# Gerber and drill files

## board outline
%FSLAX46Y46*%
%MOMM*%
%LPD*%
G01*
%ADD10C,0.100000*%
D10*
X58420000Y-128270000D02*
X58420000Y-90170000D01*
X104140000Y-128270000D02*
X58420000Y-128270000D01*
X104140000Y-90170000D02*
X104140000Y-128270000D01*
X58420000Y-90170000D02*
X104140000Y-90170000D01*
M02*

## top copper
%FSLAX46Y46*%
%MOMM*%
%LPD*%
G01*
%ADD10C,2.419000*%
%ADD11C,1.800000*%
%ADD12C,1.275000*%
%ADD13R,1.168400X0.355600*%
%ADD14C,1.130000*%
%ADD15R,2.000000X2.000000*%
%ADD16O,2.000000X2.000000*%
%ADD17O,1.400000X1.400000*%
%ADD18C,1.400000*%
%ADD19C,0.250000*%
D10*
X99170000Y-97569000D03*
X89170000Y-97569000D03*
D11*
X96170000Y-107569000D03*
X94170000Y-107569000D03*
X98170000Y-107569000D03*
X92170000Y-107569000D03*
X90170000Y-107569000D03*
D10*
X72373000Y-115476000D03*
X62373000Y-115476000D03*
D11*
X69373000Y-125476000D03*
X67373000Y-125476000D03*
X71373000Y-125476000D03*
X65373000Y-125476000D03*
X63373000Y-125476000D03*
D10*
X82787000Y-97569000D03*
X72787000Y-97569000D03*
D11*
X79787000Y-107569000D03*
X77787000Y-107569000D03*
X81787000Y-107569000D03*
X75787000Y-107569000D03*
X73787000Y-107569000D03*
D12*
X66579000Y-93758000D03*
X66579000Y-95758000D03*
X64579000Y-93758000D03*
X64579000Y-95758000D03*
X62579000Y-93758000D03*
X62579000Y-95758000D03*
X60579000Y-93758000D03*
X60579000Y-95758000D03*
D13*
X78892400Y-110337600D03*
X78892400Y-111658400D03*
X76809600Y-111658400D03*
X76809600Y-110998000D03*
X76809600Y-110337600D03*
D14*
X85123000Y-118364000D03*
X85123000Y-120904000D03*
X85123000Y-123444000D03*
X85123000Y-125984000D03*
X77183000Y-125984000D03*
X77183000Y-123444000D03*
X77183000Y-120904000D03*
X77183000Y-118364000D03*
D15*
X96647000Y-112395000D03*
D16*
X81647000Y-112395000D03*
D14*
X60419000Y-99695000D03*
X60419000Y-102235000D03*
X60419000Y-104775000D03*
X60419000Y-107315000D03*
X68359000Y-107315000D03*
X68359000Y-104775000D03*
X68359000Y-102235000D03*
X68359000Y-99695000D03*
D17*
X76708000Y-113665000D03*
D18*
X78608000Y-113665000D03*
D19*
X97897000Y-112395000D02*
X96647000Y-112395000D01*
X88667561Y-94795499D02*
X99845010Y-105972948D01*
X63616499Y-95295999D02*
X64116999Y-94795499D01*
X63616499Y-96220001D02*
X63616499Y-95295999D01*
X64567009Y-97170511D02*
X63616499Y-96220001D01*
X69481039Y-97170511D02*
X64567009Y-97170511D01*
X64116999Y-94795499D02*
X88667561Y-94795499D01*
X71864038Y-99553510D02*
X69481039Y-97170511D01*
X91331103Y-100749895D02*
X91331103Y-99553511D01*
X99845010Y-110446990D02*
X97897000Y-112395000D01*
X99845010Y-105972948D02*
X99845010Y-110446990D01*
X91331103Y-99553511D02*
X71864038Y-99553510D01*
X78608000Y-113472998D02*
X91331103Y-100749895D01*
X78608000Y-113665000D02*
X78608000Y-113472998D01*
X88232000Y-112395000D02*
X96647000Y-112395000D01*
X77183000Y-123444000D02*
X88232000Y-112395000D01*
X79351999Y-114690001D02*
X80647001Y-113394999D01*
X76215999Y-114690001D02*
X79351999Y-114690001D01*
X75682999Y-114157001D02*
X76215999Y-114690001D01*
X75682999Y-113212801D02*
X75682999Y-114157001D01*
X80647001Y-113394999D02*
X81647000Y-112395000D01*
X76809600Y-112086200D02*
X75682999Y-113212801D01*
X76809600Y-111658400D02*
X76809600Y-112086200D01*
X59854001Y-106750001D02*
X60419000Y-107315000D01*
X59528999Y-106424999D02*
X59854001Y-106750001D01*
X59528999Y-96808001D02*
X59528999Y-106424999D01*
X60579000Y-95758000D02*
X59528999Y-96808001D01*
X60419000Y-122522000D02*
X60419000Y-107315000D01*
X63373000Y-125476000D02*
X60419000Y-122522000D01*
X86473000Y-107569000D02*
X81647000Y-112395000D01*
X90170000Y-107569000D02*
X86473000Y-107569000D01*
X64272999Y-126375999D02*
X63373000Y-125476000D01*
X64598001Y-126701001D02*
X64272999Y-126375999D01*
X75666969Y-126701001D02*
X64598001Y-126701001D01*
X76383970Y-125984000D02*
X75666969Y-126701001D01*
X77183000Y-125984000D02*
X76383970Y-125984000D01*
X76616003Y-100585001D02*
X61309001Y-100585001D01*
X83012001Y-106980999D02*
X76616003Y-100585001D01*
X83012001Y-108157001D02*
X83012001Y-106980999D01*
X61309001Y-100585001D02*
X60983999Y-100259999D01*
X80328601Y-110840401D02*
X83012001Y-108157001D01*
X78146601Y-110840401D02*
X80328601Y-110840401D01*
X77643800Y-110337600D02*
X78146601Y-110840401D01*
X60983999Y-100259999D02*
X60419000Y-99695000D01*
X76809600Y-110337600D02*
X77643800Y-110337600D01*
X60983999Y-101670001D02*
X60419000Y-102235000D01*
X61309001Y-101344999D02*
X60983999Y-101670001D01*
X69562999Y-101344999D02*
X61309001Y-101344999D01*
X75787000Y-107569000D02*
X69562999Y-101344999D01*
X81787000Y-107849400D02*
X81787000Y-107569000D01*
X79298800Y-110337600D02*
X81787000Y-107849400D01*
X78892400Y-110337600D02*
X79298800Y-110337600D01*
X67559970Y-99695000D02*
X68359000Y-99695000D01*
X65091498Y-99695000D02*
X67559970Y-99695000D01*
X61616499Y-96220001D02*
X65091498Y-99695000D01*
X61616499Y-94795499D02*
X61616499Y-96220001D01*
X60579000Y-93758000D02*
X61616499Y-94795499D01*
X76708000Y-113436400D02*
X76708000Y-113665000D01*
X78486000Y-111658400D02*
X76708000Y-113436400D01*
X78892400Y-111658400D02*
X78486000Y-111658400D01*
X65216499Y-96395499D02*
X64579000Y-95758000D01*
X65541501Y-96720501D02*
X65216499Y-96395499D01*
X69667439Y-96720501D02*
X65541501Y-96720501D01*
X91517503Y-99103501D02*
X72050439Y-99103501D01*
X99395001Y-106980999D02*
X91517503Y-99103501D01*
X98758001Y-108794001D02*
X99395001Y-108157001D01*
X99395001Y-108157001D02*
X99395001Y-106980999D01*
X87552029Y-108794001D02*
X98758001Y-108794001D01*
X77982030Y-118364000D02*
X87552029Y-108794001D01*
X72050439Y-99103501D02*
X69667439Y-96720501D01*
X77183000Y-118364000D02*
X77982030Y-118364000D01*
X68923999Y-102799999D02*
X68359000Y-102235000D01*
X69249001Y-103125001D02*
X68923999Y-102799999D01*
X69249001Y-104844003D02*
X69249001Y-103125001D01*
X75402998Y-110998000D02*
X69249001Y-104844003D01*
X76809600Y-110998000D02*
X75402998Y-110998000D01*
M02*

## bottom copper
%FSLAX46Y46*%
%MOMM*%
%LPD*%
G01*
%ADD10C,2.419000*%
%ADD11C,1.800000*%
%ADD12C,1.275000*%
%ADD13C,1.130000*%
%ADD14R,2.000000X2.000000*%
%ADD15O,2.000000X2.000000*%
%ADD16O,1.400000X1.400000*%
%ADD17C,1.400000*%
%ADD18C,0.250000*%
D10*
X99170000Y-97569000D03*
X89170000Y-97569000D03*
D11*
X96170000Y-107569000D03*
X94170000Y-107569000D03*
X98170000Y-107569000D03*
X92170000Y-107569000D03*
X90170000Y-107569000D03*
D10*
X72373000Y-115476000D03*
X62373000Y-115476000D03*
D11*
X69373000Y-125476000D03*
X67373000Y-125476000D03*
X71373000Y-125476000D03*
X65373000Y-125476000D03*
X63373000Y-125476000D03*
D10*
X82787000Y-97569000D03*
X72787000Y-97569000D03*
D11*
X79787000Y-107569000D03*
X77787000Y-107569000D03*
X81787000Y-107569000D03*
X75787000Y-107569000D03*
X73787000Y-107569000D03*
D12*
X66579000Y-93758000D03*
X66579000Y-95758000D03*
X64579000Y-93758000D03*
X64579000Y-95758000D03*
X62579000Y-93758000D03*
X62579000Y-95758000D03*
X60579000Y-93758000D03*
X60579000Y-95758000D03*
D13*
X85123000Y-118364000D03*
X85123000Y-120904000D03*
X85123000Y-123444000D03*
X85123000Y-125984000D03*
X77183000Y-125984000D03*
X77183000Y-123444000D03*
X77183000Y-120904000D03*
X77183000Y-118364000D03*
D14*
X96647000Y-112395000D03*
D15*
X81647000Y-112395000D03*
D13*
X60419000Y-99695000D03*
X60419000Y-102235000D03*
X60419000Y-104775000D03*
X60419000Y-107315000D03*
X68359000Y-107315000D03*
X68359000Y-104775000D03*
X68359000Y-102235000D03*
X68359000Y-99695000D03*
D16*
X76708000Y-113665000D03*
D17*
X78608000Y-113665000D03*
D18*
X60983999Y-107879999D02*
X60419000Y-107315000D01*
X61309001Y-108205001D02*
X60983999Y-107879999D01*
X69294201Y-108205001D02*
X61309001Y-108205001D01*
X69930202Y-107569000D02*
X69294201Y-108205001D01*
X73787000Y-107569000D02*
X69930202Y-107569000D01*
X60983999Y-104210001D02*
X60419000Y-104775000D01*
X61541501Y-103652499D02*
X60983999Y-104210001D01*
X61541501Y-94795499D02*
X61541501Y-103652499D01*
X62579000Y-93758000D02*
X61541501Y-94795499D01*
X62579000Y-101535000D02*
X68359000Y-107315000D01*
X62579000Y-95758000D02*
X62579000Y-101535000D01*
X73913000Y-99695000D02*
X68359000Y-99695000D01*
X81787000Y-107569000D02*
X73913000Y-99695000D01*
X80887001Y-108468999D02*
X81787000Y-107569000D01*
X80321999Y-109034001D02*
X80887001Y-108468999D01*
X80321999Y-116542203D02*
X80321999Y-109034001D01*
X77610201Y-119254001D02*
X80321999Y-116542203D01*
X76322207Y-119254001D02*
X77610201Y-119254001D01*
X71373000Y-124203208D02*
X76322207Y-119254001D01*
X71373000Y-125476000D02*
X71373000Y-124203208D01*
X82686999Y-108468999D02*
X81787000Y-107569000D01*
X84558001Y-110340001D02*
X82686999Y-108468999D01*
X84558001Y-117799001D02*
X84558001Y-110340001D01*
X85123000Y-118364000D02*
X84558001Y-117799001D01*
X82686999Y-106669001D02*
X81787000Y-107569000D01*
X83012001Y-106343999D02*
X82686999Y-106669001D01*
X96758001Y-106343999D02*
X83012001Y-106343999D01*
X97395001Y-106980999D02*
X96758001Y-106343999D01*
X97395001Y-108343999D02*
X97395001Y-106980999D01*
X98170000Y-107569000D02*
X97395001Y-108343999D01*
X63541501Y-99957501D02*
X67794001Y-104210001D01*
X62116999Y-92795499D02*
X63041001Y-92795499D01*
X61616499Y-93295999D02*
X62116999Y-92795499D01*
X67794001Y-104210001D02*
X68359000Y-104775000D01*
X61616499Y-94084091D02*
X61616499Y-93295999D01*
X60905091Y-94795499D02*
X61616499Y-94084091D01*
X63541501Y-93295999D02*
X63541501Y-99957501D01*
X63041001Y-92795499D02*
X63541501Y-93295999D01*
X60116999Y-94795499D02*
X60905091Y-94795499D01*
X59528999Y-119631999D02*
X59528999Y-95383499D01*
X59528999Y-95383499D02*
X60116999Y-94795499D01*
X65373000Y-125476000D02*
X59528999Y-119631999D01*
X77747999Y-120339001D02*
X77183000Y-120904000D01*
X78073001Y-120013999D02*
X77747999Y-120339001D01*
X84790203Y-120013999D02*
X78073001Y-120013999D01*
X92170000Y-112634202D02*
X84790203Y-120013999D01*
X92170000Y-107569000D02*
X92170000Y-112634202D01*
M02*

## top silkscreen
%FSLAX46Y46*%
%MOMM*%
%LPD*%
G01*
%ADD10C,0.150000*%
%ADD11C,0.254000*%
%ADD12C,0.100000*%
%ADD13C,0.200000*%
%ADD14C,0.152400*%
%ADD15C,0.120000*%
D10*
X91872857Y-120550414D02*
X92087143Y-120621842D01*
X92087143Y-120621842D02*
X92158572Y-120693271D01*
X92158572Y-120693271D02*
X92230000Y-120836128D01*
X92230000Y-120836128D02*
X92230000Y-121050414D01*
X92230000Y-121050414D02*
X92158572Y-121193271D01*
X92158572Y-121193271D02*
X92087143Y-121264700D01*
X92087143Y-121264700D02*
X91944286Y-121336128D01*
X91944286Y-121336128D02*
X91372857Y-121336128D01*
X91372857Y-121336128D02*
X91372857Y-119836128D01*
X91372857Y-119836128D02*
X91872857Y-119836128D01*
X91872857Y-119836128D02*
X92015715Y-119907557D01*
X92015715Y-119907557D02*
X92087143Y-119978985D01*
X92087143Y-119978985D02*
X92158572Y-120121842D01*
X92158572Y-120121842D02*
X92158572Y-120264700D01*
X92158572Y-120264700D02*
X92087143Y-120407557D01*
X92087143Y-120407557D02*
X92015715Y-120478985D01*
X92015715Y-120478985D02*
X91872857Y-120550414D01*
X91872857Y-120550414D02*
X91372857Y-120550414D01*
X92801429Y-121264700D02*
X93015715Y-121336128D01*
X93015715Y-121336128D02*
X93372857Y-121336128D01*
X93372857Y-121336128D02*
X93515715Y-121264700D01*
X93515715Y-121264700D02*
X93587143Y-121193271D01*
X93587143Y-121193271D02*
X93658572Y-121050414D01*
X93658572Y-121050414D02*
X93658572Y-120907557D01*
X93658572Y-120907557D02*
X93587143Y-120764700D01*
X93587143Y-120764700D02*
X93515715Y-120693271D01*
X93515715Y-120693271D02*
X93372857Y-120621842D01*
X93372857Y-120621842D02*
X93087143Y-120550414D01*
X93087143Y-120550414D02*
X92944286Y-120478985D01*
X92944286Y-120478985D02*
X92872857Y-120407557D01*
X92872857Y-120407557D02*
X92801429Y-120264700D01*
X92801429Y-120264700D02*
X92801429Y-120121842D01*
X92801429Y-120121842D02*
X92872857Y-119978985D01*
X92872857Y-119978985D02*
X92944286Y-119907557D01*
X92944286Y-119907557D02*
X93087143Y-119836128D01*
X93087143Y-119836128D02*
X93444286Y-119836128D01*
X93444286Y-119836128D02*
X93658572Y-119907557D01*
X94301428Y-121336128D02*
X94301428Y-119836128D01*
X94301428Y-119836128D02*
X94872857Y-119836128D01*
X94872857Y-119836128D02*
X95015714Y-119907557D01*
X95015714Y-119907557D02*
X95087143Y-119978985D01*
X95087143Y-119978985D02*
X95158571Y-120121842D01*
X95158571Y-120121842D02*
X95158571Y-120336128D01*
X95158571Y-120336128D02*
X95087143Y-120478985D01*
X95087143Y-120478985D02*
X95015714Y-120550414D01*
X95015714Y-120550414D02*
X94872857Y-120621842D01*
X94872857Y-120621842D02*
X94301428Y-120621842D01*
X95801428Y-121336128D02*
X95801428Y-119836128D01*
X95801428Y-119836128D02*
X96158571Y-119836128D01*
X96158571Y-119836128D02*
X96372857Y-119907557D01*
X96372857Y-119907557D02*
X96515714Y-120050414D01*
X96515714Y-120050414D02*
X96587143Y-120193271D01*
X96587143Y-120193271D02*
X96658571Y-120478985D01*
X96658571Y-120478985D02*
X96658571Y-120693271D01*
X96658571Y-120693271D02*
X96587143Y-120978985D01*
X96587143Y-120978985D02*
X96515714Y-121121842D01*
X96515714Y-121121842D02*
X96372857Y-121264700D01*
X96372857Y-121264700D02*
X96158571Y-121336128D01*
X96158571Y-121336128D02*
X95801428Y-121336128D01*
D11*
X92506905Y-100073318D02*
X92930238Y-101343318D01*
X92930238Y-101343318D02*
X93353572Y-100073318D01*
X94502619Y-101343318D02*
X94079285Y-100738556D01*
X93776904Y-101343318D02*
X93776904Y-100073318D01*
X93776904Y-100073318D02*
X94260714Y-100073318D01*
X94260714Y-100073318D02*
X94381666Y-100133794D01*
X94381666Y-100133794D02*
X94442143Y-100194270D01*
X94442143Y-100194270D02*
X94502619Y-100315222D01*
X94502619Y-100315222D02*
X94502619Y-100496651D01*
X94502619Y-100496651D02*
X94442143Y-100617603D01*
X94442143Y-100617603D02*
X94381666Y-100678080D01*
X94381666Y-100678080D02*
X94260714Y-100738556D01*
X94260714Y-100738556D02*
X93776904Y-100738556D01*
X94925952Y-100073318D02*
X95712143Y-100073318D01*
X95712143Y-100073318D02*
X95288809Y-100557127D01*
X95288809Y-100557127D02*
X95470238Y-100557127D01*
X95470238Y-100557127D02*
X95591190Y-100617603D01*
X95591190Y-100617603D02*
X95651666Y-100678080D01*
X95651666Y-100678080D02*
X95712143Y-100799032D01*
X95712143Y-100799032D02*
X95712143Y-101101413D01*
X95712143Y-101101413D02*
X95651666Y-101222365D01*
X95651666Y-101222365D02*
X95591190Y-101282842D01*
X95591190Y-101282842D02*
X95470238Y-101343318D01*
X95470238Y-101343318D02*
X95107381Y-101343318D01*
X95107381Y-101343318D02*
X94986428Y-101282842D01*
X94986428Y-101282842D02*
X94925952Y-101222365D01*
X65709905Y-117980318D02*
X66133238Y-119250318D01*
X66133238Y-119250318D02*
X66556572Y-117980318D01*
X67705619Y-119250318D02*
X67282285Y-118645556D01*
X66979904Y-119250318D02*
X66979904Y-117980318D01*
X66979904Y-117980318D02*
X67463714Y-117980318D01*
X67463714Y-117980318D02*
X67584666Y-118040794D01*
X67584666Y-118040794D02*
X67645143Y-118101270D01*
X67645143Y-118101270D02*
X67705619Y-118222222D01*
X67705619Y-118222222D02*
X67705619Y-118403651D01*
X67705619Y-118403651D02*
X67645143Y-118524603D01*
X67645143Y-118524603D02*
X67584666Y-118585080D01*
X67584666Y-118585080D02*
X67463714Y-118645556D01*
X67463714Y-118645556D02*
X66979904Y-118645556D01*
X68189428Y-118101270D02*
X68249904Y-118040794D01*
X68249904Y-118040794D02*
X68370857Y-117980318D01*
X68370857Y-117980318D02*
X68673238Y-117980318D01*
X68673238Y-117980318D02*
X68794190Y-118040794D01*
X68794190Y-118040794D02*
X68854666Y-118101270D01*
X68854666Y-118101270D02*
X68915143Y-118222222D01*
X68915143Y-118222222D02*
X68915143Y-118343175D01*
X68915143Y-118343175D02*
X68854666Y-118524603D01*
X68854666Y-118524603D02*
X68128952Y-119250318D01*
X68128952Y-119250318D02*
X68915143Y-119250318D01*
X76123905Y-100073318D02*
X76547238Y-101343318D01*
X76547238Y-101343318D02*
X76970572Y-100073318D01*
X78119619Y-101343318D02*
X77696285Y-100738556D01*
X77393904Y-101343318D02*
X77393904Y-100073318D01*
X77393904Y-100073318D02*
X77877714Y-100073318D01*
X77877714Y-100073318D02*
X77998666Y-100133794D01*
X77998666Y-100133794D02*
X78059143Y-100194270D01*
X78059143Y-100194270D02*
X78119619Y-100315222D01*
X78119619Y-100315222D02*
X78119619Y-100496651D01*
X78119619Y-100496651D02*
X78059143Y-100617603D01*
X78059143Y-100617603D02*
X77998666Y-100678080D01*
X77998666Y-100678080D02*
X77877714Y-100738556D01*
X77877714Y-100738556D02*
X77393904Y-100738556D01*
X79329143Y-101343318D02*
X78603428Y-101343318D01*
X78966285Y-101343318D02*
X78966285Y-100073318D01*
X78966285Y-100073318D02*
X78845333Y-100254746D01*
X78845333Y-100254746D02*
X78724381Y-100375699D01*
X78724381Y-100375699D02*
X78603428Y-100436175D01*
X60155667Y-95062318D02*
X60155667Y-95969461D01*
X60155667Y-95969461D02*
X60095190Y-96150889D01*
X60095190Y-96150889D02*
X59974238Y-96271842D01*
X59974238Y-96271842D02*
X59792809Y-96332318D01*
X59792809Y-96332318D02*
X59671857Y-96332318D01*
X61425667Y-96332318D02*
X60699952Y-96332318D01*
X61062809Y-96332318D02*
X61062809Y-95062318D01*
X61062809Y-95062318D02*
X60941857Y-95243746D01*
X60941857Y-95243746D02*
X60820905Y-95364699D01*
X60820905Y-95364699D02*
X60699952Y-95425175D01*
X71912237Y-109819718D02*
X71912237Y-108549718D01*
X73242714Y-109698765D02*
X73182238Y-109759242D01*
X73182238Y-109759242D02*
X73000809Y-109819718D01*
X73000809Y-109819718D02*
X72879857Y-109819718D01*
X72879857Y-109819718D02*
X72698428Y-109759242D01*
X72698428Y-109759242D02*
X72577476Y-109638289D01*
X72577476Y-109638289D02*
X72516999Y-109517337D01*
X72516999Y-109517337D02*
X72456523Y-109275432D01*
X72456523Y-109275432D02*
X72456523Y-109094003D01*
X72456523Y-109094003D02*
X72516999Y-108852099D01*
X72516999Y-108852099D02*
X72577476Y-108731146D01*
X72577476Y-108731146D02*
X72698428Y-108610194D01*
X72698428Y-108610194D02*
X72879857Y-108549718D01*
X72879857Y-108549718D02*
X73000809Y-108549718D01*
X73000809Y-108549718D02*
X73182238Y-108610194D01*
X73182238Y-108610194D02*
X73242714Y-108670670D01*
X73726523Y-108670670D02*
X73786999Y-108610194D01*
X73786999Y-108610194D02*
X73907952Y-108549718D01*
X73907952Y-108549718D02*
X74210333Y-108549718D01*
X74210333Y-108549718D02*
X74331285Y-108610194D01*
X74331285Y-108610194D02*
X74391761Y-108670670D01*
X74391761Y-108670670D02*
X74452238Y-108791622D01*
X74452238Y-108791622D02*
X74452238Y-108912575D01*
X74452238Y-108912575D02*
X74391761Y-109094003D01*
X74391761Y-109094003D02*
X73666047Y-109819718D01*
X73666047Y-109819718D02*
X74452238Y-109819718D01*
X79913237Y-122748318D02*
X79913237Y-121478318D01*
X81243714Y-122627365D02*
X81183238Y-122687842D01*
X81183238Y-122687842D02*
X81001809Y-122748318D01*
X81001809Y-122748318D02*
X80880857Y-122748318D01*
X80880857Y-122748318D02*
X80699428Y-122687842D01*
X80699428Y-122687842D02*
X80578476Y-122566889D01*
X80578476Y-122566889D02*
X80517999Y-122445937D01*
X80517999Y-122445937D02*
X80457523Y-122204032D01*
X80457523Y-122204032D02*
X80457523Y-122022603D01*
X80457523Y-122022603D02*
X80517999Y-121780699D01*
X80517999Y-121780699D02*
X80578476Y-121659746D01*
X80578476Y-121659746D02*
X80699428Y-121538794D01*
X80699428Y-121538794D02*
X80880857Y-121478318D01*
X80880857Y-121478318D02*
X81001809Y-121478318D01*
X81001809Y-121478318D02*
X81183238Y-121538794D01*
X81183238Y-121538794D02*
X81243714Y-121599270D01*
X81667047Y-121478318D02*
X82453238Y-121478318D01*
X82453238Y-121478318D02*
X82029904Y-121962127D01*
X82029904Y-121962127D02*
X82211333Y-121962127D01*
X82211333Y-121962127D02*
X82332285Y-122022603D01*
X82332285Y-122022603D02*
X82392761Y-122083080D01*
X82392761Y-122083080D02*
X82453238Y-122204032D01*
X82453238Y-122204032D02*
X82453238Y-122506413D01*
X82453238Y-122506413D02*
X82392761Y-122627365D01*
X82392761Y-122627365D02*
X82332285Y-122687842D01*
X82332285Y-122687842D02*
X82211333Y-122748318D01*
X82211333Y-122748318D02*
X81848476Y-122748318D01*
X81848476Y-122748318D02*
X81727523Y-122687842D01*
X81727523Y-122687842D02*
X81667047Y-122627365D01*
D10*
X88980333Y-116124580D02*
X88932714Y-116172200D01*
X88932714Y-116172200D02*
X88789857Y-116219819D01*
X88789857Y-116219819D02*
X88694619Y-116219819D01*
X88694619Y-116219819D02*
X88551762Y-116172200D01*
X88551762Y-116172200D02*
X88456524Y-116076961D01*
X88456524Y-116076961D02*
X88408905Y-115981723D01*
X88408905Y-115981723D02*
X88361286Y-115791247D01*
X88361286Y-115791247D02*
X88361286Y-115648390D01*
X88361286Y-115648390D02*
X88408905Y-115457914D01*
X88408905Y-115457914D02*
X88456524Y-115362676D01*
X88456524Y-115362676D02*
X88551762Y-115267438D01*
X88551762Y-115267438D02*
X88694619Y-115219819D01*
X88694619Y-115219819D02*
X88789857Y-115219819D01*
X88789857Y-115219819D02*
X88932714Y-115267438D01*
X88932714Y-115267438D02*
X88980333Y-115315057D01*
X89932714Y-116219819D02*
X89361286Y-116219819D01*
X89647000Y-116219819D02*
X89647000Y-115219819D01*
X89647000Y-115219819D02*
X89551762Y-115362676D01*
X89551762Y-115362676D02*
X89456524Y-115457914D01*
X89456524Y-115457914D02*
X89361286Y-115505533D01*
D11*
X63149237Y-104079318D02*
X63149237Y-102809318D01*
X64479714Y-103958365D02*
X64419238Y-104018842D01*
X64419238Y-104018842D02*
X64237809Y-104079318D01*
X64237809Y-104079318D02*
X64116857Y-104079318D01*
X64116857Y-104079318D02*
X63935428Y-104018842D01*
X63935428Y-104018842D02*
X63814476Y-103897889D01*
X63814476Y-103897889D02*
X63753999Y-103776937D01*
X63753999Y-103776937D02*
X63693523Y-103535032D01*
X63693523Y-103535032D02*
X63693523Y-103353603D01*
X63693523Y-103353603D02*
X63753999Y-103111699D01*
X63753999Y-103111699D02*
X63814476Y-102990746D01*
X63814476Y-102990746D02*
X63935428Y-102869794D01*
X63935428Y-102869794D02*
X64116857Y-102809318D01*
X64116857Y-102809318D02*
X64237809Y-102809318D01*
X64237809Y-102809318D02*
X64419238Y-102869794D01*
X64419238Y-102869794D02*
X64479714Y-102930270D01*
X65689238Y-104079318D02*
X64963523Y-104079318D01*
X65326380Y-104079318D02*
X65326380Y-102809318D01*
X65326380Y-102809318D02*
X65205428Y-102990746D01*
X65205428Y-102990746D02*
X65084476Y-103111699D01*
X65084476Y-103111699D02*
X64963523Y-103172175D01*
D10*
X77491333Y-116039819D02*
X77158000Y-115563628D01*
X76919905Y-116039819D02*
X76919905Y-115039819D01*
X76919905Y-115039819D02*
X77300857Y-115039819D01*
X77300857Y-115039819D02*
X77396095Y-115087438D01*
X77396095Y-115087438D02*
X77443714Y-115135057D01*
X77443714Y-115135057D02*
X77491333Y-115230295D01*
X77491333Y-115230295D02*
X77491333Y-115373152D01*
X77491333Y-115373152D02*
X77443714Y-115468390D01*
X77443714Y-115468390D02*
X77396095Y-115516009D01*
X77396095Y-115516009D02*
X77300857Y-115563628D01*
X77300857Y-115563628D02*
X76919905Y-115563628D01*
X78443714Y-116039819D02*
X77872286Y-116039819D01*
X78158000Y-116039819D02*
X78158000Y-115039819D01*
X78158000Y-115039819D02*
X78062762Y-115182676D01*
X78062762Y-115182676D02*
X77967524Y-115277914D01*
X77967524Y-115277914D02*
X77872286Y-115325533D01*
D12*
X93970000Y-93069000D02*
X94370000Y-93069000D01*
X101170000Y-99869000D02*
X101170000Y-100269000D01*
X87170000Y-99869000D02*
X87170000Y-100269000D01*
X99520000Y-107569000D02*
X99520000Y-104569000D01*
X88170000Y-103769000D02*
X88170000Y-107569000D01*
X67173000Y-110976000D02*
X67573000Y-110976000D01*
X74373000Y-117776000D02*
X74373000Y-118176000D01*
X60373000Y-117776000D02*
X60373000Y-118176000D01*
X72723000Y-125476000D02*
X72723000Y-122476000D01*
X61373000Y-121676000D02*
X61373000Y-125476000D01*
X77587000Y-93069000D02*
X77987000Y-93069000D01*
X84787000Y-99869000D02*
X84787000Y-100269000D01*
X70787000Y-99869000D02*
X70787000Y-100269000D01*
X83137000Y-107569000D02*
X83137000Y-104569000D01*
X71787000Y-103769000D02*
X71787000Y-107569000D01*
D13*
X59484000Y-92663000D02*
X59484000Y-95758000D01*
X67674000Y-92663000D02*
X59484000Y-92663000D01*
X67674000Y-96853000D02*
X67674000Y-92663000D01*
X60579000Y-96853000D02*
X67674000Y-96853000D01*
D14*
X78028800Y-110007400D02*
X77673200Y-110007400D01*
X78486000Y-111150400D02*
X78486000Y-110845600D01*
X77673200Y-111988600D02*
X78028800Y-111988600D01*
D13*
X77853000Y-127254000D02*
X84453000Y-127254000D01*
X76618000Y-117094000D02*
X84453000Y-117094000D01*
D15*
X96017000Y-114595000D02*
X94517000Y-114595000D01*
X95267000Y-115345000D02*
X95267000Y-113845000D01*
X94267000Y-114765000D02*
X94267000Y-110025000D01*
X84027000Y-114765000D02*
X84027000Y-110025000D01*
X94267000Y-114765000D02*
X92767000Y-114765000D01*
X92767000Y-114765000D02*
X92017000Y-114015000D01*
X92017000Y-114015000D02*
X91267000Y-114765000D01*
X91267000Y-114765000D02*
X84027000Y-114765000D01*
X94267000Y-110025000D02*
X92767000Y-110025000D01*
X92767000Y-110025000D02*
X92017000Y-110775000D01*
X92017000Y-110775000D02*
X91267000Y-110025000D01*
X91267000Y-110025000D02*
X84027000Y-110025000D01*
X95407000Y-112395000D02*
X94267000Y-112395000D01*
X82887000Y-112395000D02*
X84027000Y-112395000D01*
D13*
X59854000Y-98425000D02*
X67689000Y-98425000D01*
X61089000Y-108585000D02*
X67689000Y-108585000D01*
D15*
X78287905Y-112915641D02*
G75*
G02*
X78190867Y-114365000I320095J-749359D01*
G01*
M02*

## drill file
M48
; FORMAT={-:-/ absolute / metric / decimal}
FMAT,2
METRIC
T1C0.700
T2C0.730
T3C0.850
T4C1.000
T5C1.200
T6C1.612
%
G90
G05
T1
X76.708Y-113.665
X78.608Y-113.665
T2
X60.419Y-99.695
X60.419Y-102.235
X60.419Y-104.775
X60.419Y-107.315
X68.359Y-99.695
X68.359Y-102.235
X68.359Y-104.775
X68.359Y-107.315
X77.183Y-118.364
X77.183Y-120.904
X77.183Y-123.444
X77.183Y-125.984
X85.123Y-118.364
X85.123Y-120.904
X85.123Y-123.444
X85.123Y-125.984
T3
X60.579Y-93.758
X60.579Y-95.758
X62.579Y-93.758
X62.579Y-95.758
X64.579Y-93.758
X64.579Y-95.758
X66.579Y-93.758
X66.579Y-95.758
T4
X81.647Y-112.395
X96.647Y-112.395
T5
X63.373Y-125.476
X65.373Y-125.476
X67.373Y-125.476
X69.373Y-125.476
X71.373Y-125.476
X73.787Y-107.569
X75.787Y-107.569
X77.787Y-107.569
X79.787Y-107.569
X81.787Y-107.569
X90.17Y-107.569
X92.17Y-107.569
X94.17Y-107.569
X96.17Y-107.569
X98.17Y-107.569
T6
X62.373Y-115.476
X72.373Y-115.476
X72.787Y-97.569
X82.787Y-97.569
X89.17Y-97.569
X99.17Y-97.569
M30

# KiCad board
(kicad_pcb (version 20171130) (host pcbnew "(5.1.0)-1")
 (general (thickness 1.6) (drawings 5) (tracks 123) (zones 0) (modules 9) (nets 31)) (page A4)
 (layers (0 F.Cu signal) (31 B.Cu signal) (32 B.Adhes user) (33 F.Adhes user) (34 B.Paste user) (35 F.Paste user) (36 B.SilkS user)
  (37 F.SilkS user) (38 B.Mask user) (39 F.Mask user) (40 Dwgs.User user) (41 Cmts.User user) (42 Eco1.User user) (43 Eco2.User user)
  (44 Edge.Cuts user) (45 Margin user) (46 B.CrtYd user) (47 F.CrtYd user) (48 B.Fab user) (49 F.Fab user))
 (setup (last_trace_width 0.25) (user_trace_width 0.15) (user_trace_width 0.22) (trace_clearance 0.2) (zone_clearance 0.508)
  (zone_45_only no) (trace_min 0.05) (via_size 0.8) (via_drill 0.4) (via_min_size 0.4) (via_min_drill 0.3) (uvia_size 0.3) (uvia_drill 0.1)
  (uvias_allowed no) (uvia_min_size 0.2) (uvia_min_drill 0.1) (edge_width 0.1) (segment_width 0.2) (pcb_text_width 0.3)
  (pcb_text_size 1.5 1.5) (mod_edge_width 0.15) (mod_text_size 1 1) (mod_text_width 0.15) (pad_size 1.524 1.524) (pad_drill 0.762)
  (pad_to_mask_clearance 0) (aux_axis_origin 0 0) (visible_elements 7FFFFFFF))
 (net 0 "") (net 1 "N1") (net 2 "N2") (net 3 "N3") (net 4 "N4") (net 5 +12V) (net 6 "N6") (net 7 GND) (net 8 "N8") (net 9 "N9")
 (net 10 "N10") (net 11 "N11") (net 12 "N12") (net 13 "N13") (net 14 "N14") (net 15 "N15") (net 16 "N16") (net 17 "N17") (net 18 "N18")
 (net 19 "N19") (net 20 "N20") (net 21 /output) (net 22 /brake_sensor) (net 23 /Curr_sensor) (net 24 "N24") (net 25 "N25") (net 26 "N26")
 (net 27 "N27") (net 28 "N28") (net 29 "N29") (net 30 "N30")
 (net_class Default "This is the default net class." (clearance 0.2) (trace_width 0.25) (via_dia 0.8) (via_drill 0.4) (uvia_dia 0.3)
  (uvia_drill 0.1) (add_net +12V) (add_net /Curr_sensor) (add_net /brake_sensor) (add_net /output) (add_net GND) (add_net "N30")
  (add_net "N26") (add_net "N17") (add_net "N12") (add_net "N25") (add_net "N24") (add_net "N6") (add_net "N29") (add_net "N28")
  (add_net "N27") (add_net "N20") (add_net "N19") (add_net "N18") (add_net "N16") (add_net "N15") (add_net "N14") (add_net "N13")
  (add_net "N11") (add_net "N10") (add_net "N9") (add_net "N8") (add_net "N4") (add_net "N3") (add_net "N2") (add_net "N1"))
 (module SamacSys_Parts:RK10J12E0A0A (layer F.Cu) (at 90.17 107.569)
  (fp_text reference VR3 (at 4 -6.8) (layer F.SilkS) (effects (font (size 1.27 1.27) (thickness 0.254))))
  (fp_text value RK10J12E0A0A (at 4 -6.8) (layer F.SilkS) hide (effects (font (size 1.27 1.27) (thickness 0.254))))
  (fp_line (start 3.8 -14.5) (end 4.2 -14.5) (layer F.SilkS) (width 0.1))
  (fp_line (start 11 -7.7) (end 11 -7.3) (layer F.SilkS) (width 0.1))
  (fp_line (start -3 -7.7) (end -3 -7.3) (layer F.SilkS) (width 0.1))
  (fp_line (start 9.35 0) (end 9.35 -3) (layer F.SilkS) (width 0.1))
  (fp_line (start -2 -3.8) (end -2 0) (layer F.SilkS) (width 0.1))
  (pad MH2 thru_hole circle (at 9 -10) (size 2.419 2.419) (drill 1.6125) (layers *.Cu *.Mask) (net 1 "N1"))
  (pad MH1 thru_hole circle (at -1 -10) (size 2.419 2.419) (drill 1.6125) (layers *.Cu *.Mask) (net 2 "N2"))
  (pad 5 thru_hole circle (at 6 0) (size 1.8 1.8) (drill 1.2) (layers *.Cu *.Mask) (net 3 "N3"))
  (pad 4 thru_hole circle (at 4 0) (size 1.8 1.8) (drill 1.2) (layers *.Cu *.Mask) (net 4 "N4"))
  (pad 3 thru_hole circle (at 8 0) (size 1.8 1.8) (drill 1.2) (layers *.Cu *.Mask) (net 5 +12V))
  (pad 2 thru_hole circle (at 2 0) (size 1.8 1.8) (drill 1.2) (layers *.Cu *.Mask) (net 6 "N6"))
  (pad 1 thru_hole circle (at 0 0) (size 1.8 1.8) (drill 1.2) (layers *.Cu *.Mask) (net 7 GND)))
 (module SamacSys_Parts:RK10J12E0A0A (layer F.Cu) (at 63.373 125.476)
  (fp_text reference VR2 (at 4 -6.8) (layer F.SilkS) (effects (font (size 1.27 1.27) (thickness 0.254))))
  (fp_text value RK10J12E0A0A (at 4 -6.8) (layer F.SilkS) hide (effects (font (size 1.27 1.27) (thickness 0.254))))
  (fp_line (start 3.8 -14.5) (end 4.2 -14.5) (layer F.SilkS) (width 0.1))
  (fp_line (start 11 -7.7) (end 11 -7.3) (layer F.SilkS) (width 0.1))
  (fp_line (start -3 -7.7) (end -3 -7.3) (layer F.SilkS) (width 0.1))
  (fp_line (start 9.35 0) (end 9.35 -3) (layer F.SilkS) (width 0.1))
  (fp_line (start -2 -3.8) (end -2 0) (layer F.SilkS) (width 0.1))
  (pad MH2 thru_hole circle (at 9 -10) (size 2.419 2.419) (drill 1.6125) (layers *.Cu *.Mask) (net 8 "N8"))
  (pad MH1 thru_hole circle (at -1 -10) (size 2.419 2.419) (drill 1.6125) (layers *.Cu *.Mask) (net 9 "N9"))
  (pad 5 thru_hole circle (at 6 0) (size 1.8 1.8) (drill 1.2) (layers *.Cu *.Mask) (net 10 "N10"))
  (pad 4 thru_hole circle (at 4 0) (size 1.8 1.8) (drill 1.2) (layers *.Cu *.Mask) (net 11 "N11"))
  (pad 3 thru_hole circle (at 8 0) (size 1.8 1.8) (drill 1.2) (layers *.Cu *.Mask) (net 5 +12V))
  (pad 2 thru_hole circle (at 2 0) (size 1.8 1.8) (drill 1.2) (layers *.Cu *.Mask) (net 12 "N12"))
  (pad 1 thru_hole circle (at 0 0) (size 1.8 1.8) (drill 1.2) (layers *.Cu *.Mask) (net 7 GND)))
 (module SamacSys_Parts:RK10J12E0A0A (layer F.Cu) (at 73.787 107.569)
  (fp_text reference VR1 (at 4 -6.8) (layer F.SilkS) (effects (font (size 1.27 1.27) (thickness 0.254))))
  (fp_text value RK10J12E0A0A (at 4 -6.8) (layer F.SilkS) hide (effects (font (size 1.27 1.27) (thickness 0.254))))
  (fp_line (start 3.8 -14.5) (end 4.2 -14.5) (layer F.SilkS) (width 0.1))
  (fp_line (start 11 -7.7) (end 11 -7.3) (layer F.SilkS) (width 0.1))
  (fp_line (start -3 -7.7) (end -3 -7.3) (layer F.SilkS) (width 0.1))
  (fp_line (start 9.35 0) (end 9.35 -3) (layer F.SilkS) (width 0.1))
  (fp_line (start -2 -3.8) (end -2 0) (layer F.SilkS) (width 0.1))
  (pad MH2 thru_hole circle (at 9 -10) (size 2.419 2.419) (drill 1.6125) (layers *.Cu *.Mask) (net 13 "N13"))
  (pad MH1 thru_hole circle (at -1 -10) (size 2.419 2.419) (drill 1.6125) (layers *.Cu *.Mask) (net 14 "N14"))
  (pad 5 thru_hole circle (at 6 0) (size 1.8 1.8) (drill 1.2) (layers *.Cu *.Mask) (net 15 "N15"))
  (pad 4 thru_hole circle (at 4 0) (size 1.8 1.8) (drill 1.2) (layers *.Cu *.Mask) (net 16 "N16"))
  (pad 3 thru_hole circle (at 8 0) (size 1.8 1.8) (drill 1.2) (layers *.Cu *.Mask) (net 5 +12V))
  (pad 2 thru_hole circle (at 2 0) (size 1.8 1.8) (drill 1.2) (layers *.Cu *.Mask) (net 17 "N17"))
  (pad 1 thru_hole circle (at 0 0) (size 1.8 1.8) (drill 1.2) (layers *.Cu *.Mask) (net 7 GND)))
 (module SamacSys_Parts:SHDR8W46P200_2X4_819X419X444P (layer F.Cu) (at 60.579 95.758)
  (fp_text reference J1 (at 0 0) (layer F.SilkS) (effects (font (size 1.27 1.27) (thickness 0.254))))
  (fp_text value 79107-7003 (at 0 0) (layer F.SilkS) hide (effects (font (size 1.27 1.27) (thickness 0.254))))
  (fp_line (start -1.095 -3.095) (end -1.095 0) (layer F.SilkS) (width 0.2))
  (fp_line (start 7.095 -3.095) (end -1.095 -3.095) (layer F.SilkS) (width 0.2))
  (fp_line (start 7.095 1.095) (end 7.095 -3.095) (layer F.SilkS) (width 0.2))
  (fp_line (start 0 1.095) (end 7.095 1.095) (layer F.SilkS) (width 0.2))
  (pad 8 thru_hole circle (at 6 -2) (size 1.275 1.275) (drill 0.85) (layers *.Cu *.Mask) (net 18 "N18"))
  (pad 7 thru_hole circle (at 6 0) (size 1.275 1.275) (drill 0.85) (layers *.Cu *.Mask) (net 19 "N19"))
  (pad 6 thru_hole circle (at 4 -2) (size 1.275 1.275) (drill 0.85) (layers *.Cu *.Mask) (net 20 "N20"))
  (pad 5 thru_hole circle (at 4 0) (size 1.275 1.275) (drill 0.85) (layers *.Cu *.Mask) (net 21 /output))
  (pad 4 thru_hole circle (at 2 -2) (size 1.275 1.275) (drill 0.85) (layers *.Cu *.Mask) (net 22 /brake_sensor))
  (pad 3 thru_hole circle (at 2 0) (size 1.275 1.275) (drill 0.85) (layers *.Cu *.Mask) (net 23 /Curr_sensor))
  (pad 2 thru_hole circle (at 0 -2) (size 1.275 1.275) (drill 0.85) (layers *.Cu *.Mask) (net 5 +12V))
  (pad 1 thru_hole circle (at 0 0) (size 1.275 1.275) (drill 0.85) (layers *.Cu *.Mask) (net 7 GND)))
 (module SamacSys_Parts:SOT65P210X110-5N (layer F.Cu) (at 77.851 110.998)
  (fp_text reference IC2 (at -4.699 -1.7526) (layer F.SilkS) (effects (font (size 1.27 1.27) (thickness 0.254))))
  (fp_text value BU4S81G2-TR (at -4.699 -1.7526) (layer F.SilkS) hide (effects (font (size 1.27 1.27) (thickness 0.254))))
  (fp_line (start 0.1778 -0.9906) (end -0.1778 -0.9906) (layer F.SilkS) (width 0.1524))
  (fp_line (start 0.635 0.1524) (end 0.635 -0.1524) (layer F.SilkS) (width 0.1524))
  (fp_line (start -0.1778 0.9906) (end 0.1778 0.9906) (layer F.SilkS) (width 0.1524))
  (pad 5 smd rect (at 1.0414 -0.6604 90) (size 0.3556 1.1684) (layers F.Cu F.Paste F.Mask) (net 5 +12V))
  (pad 4 smd rect (at 1.0414 0.6604 90) (size 0.3556 1.1684) (layers F.Cu F.Paste F.Mask) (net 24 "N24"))
  (pad 3 smd rect (at -1.0414 0.6604 90) (size 0.3556 1.1684) (layers F.Cu F.Paste F.Mask) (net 7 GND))
  (pad 2 smd rect (at -1.0414 0 90) (size 0.3556 1.1684) (layers F.Cu F.Paste F.Mask) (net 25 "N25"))
  (pad 1 smd rect (at -1.0414 -0.6604 90) (size 0.3556 1.1684) (layers F.Cu F.Paste F.Mask) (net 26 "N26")))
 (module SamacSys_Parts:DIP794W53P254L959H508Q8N (layer F.Cu) (at 81.153 122.174)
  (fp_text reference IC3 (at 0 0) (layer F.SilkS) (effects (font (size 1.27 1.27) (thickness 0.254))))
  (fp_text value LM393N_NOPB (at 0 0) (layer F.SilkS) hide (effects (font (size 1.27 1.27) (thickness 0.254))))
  (fp_line (start -3.3 5.08) (end 3.3 5.08) (layer F.SilkS) (width 0.2))
  (fp_line (start -4.535 -5.08) (end 3.3 -5.08) (layer F.SilkS) (width 0.2))
  (pad 8 thru_hole circle (at 3.97 -3.81) (size 1.13 1.13) (drill 0.73) (layers *.Cu *.Mask) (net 5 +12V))
  (pad 7 thru_hole circle (at 3.97 -1.27) (size 1.13 1.13) (drill 0.73) (layers *.Cu *.Mask) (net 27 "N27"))
  (pad 6 thru_hole circle (at 3.97 1.27) (size 1.13 1.13) (drill 0.73) (layers *.Cu *.Mask) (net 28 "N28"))
  (pad 5 thru_hole circle (at 3.97 3.81) (size 1.13 1.13) (drill 0.73) (layers *.Cu *.Mask) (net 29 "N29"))
  (pad 4 thru_hole circle (at -3.97 3.81) (size 1.13 1.13) (drill 0.73) (layers *.Cu *.Mask) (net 7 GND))
  (pad 3 thru_hole circle (at -3.97 1.27) (size 1.13 1.13) (drill 0.73) (layers *.Cu *.Mask) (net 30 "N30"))
  (pad 2 thru_hole circle (at -3.97 -1.27) (size 1.13 1.13) (drill 0.73) (layers *.Cu *.Mask) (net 6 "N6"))
  (pad 1 thru_hole circle (at -3.97 -3.81) (size 1.13 1.13) (drill 0.73) (layers *.Cu *.Mask) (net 21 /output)))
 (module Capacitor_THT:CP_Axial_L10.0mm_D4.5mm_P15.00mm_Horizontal (layer F.Cu) (at 96.647 112.395 180)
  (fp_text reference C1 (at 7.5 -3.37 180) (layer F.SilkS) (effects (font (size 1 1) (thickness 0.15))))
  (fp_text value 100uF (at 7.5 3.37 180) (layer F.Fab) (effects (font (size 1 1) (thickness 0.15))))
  (fp_line (start 0.63 -2.2) (end 2.13 -2.2) (layer F.SilkS) (width 0.12))
  (fp_line (start 1.38 -2.95) (end 1.38 -1.45) (layer F.SilkS) (width 0.12))
  (fp_line (start 2.38 -2.37) (end 2.38 2.37) (layer F.SilkS) (width 0.12))
  (fp_line (start 12.62 -2.37) (end 12.62 2.37) (layer F.SilkS) (width 0.12))
  (fp_line (start 2.38 -2.37) (end 3.88 -2.37) (layer F.SilkS) (width 0.12))
  (fp_line (start 3.88 -2.37) (end 4.63 -1.62) (layer F.SilkS) (width 0.12))
  (fp_line (start 4.63 -1.62) (end 5.38 -2.37) (layer F.SilkS) (width 0.12))
  (fp_line (start 5.38 -2.37) (end 12.62 -2.37) (layer F.SilkS) (width 0.12))
  (fp_line (start 2.38 2.37) (end 3.88 2.37) (layer F.SilkS) (width 0.12))
  (fp_line (start 3.88 2.37) (end 4.63 1.62) (layer F.SilkS) (width 0.12))
  (fp_line (start 4.63 1.62) (end 5.38 2.37) (layer F.SilkS) (width 0.12))
  (fp_line (start 5.38 2.37) (end 12.62 2.37) (layer F.SilkS) (width 0.12))
  (fp_line (start 1.24 0) (end 2.38 0) (layer F.SilkS) (width 0.12))
  (fp_line (start 13.76 0) (end 12.62 0) (layer F.SilkS) (width 0.12))
  (pad 1 thru_hole rect (at 0 0 180) (size 2 2) (drill 1) (layers *.Cu *.Mask) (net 30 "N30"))
  (pad 2 thru_hole oval (at 15 0 180) (size 2 2) (drill 1) (layers *.Cu *.Mask) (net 7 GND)))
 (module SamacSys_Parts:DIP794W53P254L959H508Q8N (layer F.Cu) (at 64.389 103.505)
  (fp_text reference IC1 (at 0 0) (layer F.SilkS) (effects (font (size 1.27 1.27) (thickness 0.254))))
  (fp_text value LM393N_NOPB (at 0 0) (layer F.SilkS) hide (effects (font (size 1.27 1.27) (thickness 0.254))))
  (fp_line (start -4.535 -5.08) (end 3.3 -5.08) (layer F.SilkS) (width 0.2))
  (fp_line (start -3.3 5.08) (end 3.3 5.08) (layer F.SilkS) (width 0.2))
  (pad 1 thru_hole circle (at -3.97 -3.81) (size 1.13 1.13) (drill 0.73) (layers *.Cu *.Mask) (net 26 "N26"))
  (pad 2 thru_hole circle (at -3.97 -1.27) (size 1.13 1.13) (drill 0.73) (layers *.Cu *.Mask) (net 17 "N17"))
  (pad 3 thru_hole circle (at -3.97 1.27) (size 1.13 1.13) (drill 0.73) (layers *.Cu *.Mask) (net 22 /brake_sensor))
  (pad 4 thru_hole circle (at -3.97 3.81) (size 1.13 1.13) (drill 0.73) (layers *.Cu *.Mask) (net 7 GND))
  (pad 5 thru_hole circle (at 3.97 3.81) (size 1.13 1.13) (drill 0.73) (layers *.Cu *.Mask) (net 23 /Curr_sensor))
  (pad 6 thru_hole circle (at 3.97 1.27) (size 1.13 1.13) (drill 0.73) (layers *.Cu *.Mask) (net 12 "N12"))
  (pad 7 thru_hole circle (at 3.97 -1.27) (size 1.13 1.13) (drill 0.73) (layers *.Cu *.Mask) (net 25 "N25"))
  (pad 8 thru_hole circle (at 3.97 -3.81) (size 1.13 1.13) (drill 0.73) (layers *.Cu *.Mask) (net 5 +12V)))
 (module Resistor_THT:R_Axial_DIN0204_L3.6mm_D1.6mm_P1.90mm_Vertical (layer F.Cu) (at 78.608 113.665 180)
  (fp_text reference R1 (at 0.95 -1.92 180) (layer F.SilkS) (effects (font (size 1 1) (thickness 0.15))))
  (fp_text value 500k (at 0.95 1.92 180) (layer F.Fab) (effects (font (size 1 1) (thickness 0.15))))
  (fp_arc (start 0 0) (end 0.417133 -0.7) (angle -233.92106) (layer F.SilkS) (width 0.12))
  (pad 2 thru_hole oval (at 1.9 0 180) (size 1.4 1.4) (drill 0.7) (layers *.Cu *.Mask) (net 24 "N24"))
  (pad 1 thru_hole circle (at 0 0 180) (size 1.4 1.4) (drill 0.7) (layers *.Cu *.Mask) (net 30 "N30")))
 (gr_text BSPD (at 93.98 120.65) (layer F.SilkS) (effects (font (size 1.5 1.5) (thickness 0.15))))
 (gr_line (start 58.42 128.27) (end 58.42 90.17) (layer Edge.Cuts) (width 0.1))
 (gr_line (start 104.14 128.27) (end 58.42 128.27) (layer Edge.Cuts) (width 0.1))
 (gr_line (start 104.14 90.17) (end 104.14 128.27) (layer Edge.Cuts) (width 0.1))
 (gr_line (start 58.42 90.17) (end 104.14 90.17) (layer Edge.Cuts) (width 0.1))
 (segment (start 97.897 112.395) (end 96.647 112.395) (width 0.25) (layer F.Cu) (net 30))
 (segment (start 88.667561 94.795499) (end 99.84501 105.972948) (width 0.25) (layer F.Cu) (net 30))
 (segment (start 63.616499 95.295999) (end 64.116999 94.795499) (width 0.25) (layer F.Cu) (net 30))
 (segment (start 63.616499 96.220001) (end 63.616499 95.295999) (width 0.25) (layer F.Cu) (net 30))
 (segment (start 64.567009 97.170511) (end 63.616499 96.220001) (width 0.25) (layer F.Cu) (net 30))
 (segment (start 69.481039 97.170511) (end 64.567009 97.170511) (width 0.25) (layer F.Cu) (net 30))
 (segment (start 64.116999 94.795499) (end 88.667561 94.795499) (width 0.25) (layer F.Cu) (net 30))
 (segment (start 71.864038 99.55351) (end 69.481039 97.170511) (width 0.25) (layer F.Cu) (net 30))
 (segment (start 91.331103 100.749895) (end 91.331103 99.553511) (width 0.25) (layer F.Cu) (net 30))
 (segment (start 99.84501 110.44699) (end 97.897 112.395) (width 0.25) (layer F.Cu) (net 30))
 (segment (start 99.84501 105.972948) (end 99.84501 110.44699) (width 0.25) (layer F.Cu) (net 30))
 (segment (start 91.331103 99.553511) (end 71.864038 99.55351) (width 0.25) (layer F.Cu) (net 30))
 (segment (start 78.608 113.472998) (end 91.331103 100.749895) (width 0.25) (layer F.Cu) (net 30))
 (segment (start 78.608 113.665) (end 78.608 113.472998) (width 0.25) (layer F.Cu) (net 30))
 (segment (start 88.232 112.395) (end 96.647 112.395) (width 0.25) (layer F.Cu) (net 30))
 (segment (start 77.183 123.444) (end 88.232 112.395) (width 0.25) (layer F.Cu) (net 30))
 (segment (start 79.351999 114.690001) (end 80.647001 113.394999) (width 0.25) (layer F.Cu) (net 7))
 (segment (start 76.215999 114.690001) (end 79.351999 114.690001) (width 0.25) (layer F.Cu) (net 7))
 (segment (start 75.682999 114.157001) (end 76.215999 114.690001) (width 0.25) (layer F.Cu) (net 7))
 (segment (start 75.682999 113.212801) (end 75.682999 114.157001) (width 0.25) (layer F.Cu) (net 7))
 (segment (start 80.647001 113.394999) (end 81.647 112.395) (width 0.25) (layer F.Cu) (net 7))
 (segment (start 76.8096 112.0862) (end 75.682999 113.212801) (width 0.25) (layer F.Cu) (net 7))
 (segment (start 76.8096 111.6584) (end 76.8096 112.0862) (width 0.25) (layer F.Cu) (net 7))
 (segment (start 59.854001 106.750001) (end 60.419 107.315) (width 0.25) (layer F.Cu) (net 7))
 (segment (start 59.528999 106.424999) (end 59.854001 106.750001) (width 0.25) (layer F.Cu) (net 7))
 (segment (start 59.528999 96.808001) (end 59.528999 106.424999) (width 0.25) (layer F.Cu) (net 7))
 (segment (start 60.579 95.758) (end 59.528999 96.808001) (width 0.25) (layer F.Cu) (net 7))
 (segment (start 60.983999 107.879999) (end 60.419 107.315) (width 0.25) (layer B.Cu) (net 7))
 (segment (start 61.309001 108.205001) (end 60.983999 107.879999) (width 0.25) (layer B.Cu) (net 7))
 (segment (start 69.294201 108.205001) (end 61.309001 108.205001) (width 0.25) (layer B.Cu) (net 7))
 (segment (start 69.930202 107.569) (end 69.294201 108.205001) (width 0.25) (layer B.Cu) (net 7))
 (segment (start 73.787 107.569) (end 69.930202 107.569) (width 0.25) (layer B.Cu) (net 7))
 (segment (start 60.419 122.522) (end 60.419 107.315) (width 0.25) (layer F.Cu) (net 7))
 (segment (start 63.373 125.476) (end 60.419 122.522) (width 0.25) (layer F.Cu) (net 7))
 (segment (start 86.473 107.569) (end 81.647 112.395) (width 0.25) (layer F.Cu) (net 7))
 (segment (start 90.17 107.569) (end 86.473 107.569) (width 0.25) (layer F.Cu) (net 7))
 (segment (start 64.272999 126.375999) (end 63.373 125.476) (width 0.25) (layer F.Cu) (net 7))
 (segment (start 64.598001 126.701001) (end 64.272999 126.375999) (width 0.25) (layer F.Cu) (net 7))
 (segment (start 75.666969 126.701001) (end 64.598001 126.701001) (width 0.25) (layer F.Cu) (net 7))
 (segment (start 76.38397 125.984) (end 75.666969 126.701001) (width 0.25) (layer F.Cu) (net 7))
 (segment (start 77.183 125.984) (end 76.38397 125.984) (width 0.25) (layer F.Cu) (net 7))
 (segment (start 76.616003 100.585001) (end 61.309001 100.585001) (width 0.25) (layer F.Cu) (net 26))
 (segment (start 83.012001 106.980999) (end 76.616003 100.585001) (width 0.25) (layer F.Cu) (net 26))
 (segment (start 83.012001 108.157001) (end 83.012001 106.980999) (width 0.25) (layer F.Cu) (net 26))
 (segment (start 61.309001 100.585001) (end 60.983999 100.259999) (width 0.25) (layer F.Cu) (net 26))
 (segment (start 80.328601 110.840401) (end 83.012001 108.157001) (width 0.25) (layer F.Cu) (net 26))
 (segment (start 78.146601 110.840401) (end 80.328601 110.840401) (width 0.25) (layer F.Cu) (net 26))
 (segment (start 77.6438 110.3376) (end 78.146601 110.840401) (width 0.25) (layer F.Cu) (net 26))
 (segment (start 60.983999 100.259999) (end 60.419 99.695) (width 0.25) (layer F.Cu) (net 26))
 (segment (start 76.8096 110.3376) (end 77.6438 110.3376) (width 0.25) (layer F.Cu) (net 26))
 (segment (start 60.983999 101.670001) (end 60.419 102.235) (width 0.25) (layer F.Cu) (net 17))
 (segment (start 61.309001 101.344999) (end 60.983999 101.670001) (width 0.25) (layer F.Cu) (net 17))
 (segment (start 69.562999 101.344999) (end 61.309001 101.344999) (width 0.25) (layer F.Cu) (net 17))
 (segment (start 75.787 107.569) (end 69.562999 101.344999) (width 0.25) (layer F.Cu) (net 17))
 (segment (start 60.983999 104.210001) (end 60.419 104.775) (width 0.25) (layer B.Cu) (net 22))
 (segment (start 61.541501 103.652499) (end 60.983999 104.210001) (width 0.25) (layer B.Cu) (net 22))
 (segment (start 61.541501 94.795499) (end 61.541501 103.652499) (width 0.25) (layer B.Cu) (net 22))
 (segment (start 62.579 93.758) (end 61.541501 94.795499) (width 0.25) (layer B.Cu) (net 22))
 (segment (start 62.579 101.535) (end 68.359 107.315) (width 0.25) (layer B.Cu) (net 23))
 (segment (start 62.579 95.758) (end 62.579 101.535) (width 0.25) (layer B.Cu) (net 23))
 (segment (start 81.787 107.8494) (end 81.787 107.569) (width 0.25) (layer F.Cu) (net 5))
 (segment (start 79.2988 110.3376) (end 81.787 107.8494) (width 0.25) (layer F.Cu) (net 5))
 (segment (start 78.8924 110.3376) (end 79.2988 110.3376) (width 0.25) (layer F.Cu) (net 5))
 (segment (start 67.55997 99.695) (end 68.359 99.695) (width 0.25) (layer F.Cu) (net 5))
 (segment (start 65.091498 99.695) (end 67.55997 99.695) (width 0.25) (layer F.Cu) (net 5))
 (segment (start 61.616499 96.220001) (end 65.091498 99.695) (width 0.25) (layer F.Cu) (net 5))
 (segment (start 61.616499 94.795499) (end 61.616499 96.220001) (width 0.25) (layer F.Cu) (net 5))
 (segment (start 60.579 93.758) (end 61.616499 94.795499) (width 0.25) (layer F.Cu) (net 5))
 (segment (start 73.913 99.695) (end 68.359 99.695) (width 0.25) (layer B.Cu) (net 5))
 (segment (start 81.787 107.569) (end 73.913 99.695) (width 0.25) (layer B.Cu) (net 5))
 (segment (start 80.887001 108.468999) (end 81.787 107.569) (width 0.25) (layer B.Cu) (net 5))
 (segment (start 80.321999 109.034001) (end 80.887001 108.468999) (width 0.25) (layer B.Cu) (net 5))
 (segment (start 80.321999 116.542203) (end 80.321999 109.034001) (width 0.25) (layer B.Cu) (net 5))
 (segment (start 77.610201 119.254001) (end 80.321999 116.542203) (width 0.25) (layer B.Cu) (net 5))
 (segment (start 76.322207 119.254001) (end 77.610201 119.254001) (width 0.25) (layer B.Cu) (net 5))
 (segment (start 71.373 124.203208) (end 76.322207 119.254001) (width 0.25) (layer B.Cu) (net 5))
 (segment (start 71.373 125.476) (end 71.373 124.203208) (width 0.25) (layer B.Cu) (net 5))
 (segment (start 82.686999 108.468999) (end 81.787 107.569) (width 0.25) (layer B.Cu) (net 5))
 (segment (start 84.558001 110.340001) (end 82.686999 108.468999) (width 0.25) (layer B.Cu) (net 5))
 (segment (start 84.558001 117.799001) (end 84.558001 110.340001) (width 0.25) (layer B.Cu) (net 5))
 (segment (start 85.123 118.364) (end 84.558001 117.799001) (width 0.25) (layer B.Cu) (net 5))
 (segment (start 82.686999 106.669001) (end 81.787 107.569) (width 0.25) (layer B.Cu) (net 5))
 (segment (start 83.012001 106.343999) (end 82.686999 106.669001) (width 0.25) (layer B.Cu) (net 5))
 (segment (start 96.758001 106.343999) (end 83.012001 106.343999) (width 0.25) (layer B.Cu) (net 5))
 (segment (start 97.395001 106.980999) (end 96.758001 106.343999) (width 0.25) (layer B.Cu) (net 5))
 (segment (start 97.395001 108.343999) (end 97.395001 106.980999) (width 0.25) (layer B.Cu) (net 5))
 (segment (start 98.17 107.569) (end 97.395001 108.343999) (width 0.25) (layer B.Cu) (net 5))
 (segment (start 76.708 113.4364) (end 76.708 113.665) (width 0.25) (layer F.Cu) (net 24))
 (segment (start 78.486 111.6584) (end 76.708 113.4364) (width 0.25) (layer F.Cu) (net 24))
 (segment (start 78.8924 111.6584) (end 78.486 111.6584) (width 0.25) (layer F.Cu) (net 24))
 (segment (start 65.216499 96.395499) (end 64.579 95.758) (width 0.25) (layer F.Cu) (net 21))
 (segment (start 65.541501 96.720501) (end 65.216499 96.395499) (width 0.25) (layer F.Cu) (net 21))
 (segment (start 69.667439 96.720501) (end 65.541501 96.720501) (width 0.25) (layer F.Cu) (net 21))
 (segment (start 91.517503 99.103501) (end 72.050439 99.103501) (width 0.25) (layer F.Cu) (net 21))
 (segment (start 99.395001 106.980999) (end 91.517503 99.103501) (width 0.25) (layer F.Cu) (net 21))
 (segment (start 98.758001 108.794001) (end 99.395001 108.157001) (width 0.25) (layer F.Cu) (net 21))
 (segment (start 99.395001 108.157001) (end 99.395001 106.980999) (width 0.25) (layer F.Cu) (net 21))
 (segment (start 87.552029 108.794001) (end 98.758001 108.794001) (width 0.25) (layer F.Cu) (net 21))
 (segment (start 77.98203 118.364) (end 87.552029 108.794001) (width 0.25) (layer F.Cu) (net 21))
 (segment (start 72.050439 99.103501) (end 69.667439 96.720501) (width 0.25) (layer F.Cu) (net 21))
 (segment (start 77.183 118.364) (end 77.98203 118.364) (width 0.25) (layer F.Cu) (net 21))
 (segment (start 63.541501 99.957501) (end 67.794001 104.210001) (width 0.25) (layer B.Cu) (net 12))
 (segment (start 62.116999 92.795499) (end 63.041001 92.795499) (width 0.25) (layer B.Cu) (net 12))
 (segment (start 61.616499 93.295999) (end 62.116999 92.795499) (width 0.25) (layer B.Cu) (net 12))
 (segment (start 67.794001 104.210001) (end 68.359 104.775) (width 0.25) (layer B.Cu) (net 12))
 (segment (start 61.616499 94.084091) (end 61.616499 93.295999) (width 0.25) (layer B.Cu) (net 12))
 (segment (start 60.905091 94.795499) (end 61.616499 94.084091) (width 0.25) (layer B.Cu) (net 12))
 (segment (start 63.541501 93.295999) (end 63.541501 99.957501) (width 0.25) (layer B.Cu) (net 12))
 (segment (start 63.041001 92.795499) (end 63.541501 93.295999) (width 0.25) (layer B.Cu) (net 12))
 (segment (start 60.116999 94.795499) (end 60.905091 94.795499) (width 0.25) (layer B.Cu) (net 12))
 (segment (start 59.528999 119.631999) (end 59.528999 95.383499) (width 0.25) (layer B.Cu) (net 12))
 (segment (start 59.528999 95.383499) (end 60.116999 94.795499) (width 0.25) (layer B.Cu) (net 12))
 (segment (start 65.373 125.476) (end 59.528999 119.631999) (width 0.25) (layer B.Cu) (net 12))
 (segment (start 68.923999 102.799999) (end 68.359 102.235) (width 0.25) (layer F.Cu) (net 25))
 (segment (start 69.249001 103.125001) (end 68.923999 102.799999) (width 0.25) (layer F.Cu) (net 25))
 (segment (start 69.249001 104.844003) (end 69.249001 103.125001) (width 0.25) (layer F.Cu) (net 25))
 (segment (start 75.402998 110.998) (end 69.249001 104.844003) (width 0.25) (layer F.Cu) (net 25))
 (segment (start 76.8096 110.998) (end 75.402998 110.998) (width 0.25) (layer F.Cu) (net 25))
 (segment (start 77.747999 120.339001) (end 77.183 120.904) (width 0.25) (layer B.Cu) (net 6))
 (segment (start 78.073001 120.013999) (end 77.747999 120.339001) (width 0.25) (layer B.Cu) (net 6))
 (segment (start 84.790203 120.013999) (end 78.073001 120.013999) (width 0.25) (layer B.Cu) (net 6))
 (segment (start 92.17 112.634202) (end 84.790203 120.013999) (width 0.25) (layer B.Cu) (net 6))
 (segment (start 92.17 107.569) (end 92.17 112.634202) (width 0.25) (layer B.Cu) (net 6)))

